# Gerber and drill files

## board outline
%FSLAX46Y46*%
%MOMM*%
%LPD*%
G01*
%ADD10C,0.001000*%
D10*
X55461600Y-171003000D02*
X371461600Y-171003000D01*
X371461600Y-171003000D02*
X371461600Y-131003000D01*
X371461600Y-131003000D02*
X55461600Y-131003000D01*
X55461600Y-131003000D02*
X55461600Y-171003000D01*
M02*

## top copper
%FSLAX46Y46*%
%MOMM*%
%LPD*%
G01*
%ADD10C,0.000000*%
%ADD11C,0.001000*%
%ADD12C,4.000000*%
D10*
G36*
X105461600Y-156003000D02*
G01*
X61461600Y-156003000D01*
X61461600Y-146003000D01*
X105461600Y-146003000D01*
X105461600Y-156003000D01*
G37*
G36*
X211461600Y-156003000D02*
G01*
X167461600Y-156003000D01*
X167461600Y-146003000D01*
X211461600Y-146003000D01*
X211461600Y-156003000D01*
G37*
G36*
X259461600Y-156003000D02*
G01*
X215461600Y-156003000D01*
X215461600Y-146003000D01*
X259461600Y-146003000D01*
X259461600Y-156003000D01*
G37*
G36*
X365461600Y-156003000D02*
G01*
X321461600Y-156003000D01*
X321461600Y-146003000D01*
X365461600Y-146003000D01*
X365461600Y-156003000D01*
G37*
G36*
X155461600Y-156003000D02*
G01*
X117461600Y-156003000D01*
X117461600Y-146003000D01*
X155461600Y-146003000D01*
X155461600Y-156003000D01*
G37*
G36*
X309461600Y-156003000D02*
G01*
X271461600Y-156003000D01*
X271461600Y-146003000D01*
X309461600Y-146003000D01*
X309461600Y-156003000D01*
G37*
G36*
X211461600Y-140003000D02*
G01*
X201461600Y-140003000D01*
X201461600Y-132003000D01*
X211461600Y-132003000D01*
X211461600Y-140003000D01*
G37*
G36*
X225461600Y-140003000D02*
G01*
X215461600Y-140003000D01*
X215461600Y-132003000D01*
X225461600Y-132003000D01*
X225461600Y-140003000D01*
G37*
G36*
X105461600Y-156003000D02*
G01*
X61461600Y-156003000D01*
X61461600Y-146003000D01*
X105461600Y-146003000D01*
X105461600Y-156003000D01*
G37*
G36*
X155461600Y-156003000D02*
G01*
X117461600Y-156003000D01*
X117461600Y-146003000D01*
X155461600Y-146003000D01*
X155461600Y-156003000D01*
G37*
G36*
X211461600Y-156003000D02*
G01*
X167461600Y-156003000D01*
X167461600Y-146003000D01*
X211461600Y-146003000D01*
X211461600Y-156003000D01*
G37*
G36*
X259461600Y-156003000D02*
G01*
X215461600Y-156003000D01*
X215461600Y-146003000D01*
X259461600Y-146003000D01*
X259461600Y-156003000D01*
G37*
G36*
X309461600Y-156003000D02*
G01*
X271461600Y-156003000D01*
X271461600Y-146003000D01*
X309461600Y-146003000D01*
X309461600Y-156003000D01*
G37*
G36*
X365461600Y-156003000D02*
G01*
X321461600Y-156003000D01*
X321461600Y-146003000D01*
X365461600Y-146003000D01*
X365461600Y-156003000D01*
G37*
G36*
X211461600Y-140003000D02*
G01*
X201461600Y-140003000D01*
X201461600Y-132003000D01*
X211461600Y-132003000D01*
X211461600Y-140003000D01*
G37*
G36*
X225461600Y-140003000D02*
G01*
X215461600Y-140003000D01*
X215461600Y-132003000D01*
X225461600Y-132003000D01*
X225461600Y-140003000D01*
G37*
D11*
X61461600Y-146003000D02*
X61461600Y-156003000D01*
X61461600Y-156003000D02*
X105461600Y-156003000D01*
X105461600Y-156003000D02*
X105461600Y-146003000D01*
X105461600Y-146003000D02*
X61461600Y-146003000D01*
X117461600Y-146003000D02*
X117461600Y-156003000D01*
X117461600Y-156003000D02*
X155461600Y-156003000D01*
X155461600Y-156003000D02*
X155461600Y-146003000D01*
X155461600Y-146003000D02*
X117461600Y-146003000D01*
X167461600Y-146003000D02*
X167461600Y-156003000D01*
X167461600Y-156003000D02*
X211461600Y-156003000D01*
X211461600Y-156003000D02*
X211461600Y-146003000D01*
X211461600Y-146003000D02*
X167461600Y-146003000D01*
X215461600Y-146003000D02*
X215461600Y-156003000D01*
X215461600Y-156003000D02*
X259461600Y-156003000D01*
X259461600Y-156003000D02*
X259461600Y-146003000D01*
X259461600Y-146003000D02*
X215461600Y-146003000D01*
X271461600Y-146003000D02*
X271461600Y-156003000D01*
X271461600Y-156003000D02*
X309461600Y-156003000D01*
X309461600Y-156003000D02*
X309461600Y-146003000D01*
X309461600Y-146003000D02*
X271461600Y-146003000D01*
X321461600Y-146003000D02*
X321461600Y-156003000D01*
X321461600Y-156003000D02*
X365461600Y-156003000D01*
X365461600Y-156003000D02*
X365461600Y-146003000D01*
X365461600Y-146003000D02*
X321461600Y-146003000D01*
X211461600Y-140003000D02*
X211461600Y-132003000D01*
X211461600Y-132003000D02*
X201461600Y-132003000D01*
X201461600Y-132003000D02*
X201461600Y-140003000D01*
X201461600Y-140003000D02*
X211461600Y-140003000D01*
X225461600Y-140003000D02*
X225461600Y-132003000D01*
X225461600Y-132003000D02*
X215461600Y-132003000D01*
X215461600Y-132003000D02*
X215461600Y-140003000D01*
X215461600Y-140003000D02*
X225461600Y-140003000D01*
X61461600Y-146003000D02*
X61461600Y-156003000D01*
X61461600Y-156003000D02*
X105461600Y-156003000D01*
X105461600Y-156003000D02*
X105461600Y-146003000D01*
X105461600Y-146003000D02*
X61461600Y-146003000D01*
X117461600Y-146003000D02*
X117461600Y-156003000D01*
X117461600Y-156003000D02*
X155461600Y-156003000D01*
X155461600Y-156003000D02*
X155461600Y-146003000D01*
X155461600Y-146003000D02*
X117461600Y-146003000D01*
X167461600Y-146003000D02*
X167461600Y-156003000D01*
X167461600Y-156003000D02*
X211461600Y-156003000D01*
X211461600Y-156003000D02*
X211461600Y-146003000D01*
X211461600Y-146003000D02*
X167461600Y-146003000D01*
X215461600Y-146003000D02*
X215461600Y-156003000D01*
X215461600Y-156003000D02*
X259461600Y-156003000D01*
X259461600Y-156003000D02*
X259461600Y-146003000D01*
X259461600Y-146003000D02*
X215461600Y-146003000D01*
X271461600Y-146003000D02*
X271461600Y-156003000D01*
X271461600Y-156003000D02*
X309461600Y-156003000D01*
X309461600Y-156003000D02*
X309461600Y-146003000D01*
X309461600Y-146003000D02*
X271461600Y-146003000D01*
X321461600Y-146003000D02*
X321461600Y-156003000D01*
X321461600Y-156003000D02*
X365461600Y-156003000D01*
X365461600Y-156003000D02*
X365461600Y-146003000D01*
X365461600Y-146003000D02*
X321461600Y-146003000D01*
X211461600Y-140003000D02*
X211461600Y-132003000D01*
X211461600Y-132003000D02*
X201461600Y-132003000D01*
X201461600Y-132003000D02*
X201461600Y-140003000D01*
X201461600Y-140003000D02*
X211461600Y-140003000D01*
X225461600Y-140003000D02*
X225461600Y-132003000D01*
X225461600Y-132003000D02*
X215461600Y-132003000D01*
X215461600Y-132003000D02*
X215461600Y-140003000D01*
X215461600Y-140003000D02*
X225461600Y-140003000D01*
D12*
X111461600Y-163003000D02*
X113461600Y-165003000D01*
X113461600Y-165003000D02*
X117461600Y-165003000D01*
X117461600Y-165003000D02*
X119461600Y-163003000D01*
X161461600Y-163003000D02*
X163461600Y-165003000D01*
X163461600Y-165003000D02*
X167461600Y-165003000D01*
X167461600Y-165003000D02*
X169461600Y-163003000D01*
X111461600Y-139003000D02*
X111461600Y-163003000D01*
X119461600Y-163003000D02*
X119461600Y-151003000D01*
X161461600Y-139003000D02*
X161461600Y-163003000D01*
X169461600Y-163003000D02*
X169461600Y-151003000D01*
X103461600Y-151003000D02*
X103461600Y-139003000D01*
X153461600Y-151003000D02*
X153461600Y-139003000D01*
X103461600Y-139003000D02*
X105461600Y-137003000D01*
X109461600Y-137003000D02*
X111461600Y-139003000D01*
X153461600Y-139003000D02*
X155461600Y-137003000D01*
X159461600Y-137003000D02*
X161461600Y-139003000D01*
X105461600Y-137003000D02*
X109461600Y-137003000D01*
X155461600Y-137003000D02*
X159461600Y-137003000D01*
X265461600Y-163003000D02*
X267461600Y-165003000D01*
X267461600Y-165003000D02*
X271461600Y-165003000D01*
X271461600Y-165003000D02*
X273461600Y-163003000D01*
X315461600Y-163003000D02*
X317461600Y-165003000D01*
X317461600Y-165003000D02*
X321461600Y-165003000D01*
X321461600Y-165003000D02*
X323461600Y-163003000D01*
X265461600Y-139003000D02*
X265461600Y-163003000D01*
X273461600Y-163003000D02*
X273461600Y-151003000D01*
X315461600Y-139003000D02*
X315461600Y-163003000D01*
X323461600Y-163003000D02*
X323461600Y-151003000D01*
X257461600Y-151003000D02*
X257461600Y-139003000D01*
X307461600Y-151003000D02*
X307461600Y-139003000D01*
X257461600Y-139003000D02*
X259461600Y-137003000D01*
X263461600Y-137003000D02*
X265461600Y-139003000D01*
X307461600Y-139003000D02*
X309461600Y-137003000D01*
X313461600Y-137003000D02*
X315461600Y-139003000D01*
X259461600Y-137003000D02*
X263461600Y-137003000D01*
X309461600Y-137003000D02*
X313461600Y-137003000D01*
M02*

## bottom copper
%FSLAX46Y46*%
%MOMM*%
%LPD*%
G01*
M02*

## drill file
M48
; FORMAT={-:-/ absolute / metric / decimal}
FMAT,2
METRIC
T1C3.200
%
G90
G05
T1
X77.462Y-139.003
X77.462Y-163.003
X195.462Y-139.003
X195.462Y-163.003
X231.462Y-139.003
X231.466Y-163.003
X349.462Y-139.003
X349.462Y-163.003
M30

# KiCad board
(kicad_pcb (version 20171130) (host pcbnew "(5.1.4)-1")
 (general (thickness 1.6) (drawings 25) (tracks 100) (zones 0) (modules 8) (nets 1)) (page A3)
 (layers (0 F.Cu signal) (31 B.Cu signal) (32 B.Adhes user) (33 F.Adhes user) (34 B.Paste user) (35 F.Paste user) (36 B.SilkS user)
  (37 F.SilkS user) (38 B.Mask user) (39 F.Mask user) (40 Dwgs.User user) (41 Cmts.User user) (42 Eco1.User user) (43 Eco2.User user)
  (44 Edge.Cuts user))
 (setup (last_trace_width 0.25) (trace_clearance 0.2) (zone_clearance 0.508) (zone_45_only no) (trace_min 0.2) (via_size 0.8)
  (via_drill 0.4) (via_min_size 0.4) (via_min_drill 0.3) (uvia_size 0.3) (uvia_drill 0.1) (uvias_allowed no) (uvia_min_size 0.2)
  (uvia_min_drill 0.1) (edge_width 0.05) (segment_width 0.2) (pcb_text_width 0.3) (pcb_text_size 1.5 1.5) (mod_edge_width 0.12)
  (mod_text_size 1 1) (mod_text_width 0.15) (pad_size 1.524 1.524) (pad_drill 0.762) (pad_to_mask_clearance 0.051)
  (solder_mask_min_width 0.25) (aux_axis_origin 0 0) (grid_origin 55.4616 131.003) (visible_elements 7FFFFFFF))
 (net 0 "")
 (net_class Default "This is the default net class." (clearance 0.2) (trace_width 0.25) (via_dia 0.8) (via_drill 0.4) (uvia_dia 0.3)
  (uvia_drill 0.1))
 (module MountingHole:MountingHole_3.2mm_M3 (layer F.Cu) (at 349.4616 139.003)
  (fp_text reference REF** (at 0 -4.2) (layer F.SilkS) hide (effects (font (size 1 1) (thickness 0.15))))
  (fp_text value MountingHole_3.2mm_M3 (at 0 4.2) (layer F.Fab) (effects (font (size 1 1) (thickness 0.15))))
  (pad 1 np_thru_hole circle (at 0 0) (size 3.2 3.2) (drill 3.2) (layers *.Cu *.Mask)))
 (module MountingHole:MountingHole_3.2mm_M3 (layer F.Cu) (at 349.4616 163.003)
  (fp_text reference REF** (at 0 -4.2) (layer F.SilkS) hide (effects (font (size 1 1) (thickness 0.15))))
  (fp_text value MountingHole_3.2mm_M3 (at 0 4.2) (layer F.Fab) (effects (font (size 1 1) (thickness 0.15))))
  (pad 1 np_thru_hole circle (at 0 0) (size 3.2 3.2) (drill 3.2) (layers *.Cu *.Mask)))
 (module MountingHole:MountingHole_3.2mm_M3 (layer F.Cu) (at 195.4616 139.003)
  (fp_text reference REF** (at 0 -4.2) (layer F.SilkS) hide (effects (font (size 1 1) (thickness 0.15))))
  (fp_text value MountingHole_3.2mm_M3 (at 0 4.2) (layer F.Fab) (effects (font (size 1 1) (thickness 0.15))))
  (pad 1 np_thru_hole circle (at 0 0) (size 3.2 3.2) (drill 3.2) (layers *.Cu *.Mask)))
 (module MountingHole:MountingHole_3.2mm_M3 (layer F.Cu) (at 231.4616 139.003)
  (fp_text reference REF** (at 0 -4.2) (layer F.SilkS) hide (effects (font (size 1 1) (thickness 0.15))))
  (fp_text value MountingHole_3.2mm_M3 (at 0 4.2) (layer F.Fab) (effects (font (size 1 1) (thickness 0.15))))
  (pad 1 np_thru_hole circle (at 0 0) (size 3.2 3.2) (drill 3.2) (layers *.Cu *.Mask)))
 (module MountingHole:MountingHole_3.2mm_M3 (layer F.Cu) (at 231.4661 163.003)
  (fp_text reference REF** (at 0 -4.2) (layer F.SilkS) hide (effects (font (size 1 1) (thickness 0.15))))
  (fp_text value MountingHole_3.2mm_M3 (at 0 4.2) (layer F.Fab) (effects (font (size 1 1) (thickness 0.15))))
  (pad 1 np_thru_hole circle (at 0 0) (size 3.2 3.2) (drill 3.2) (layers *.Cu *.Mask)))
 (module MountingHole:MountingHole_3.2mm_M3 (layer F.Cu) (at 195.4616 163.003)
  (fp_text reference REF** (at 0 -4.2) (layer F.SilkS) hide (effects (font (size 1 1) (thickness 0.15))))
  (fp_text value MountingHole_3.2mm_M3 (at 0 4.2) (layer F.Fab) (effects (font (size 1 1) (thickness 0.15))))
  (pad 1 np_thru_hole circle (at 0 0) (size 3.2 3.2) (drill 3.2) (layers *.Cu *.Mask)))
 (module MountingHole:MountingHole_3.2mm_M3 (layer F.Cu) (at 77.4616 163.003)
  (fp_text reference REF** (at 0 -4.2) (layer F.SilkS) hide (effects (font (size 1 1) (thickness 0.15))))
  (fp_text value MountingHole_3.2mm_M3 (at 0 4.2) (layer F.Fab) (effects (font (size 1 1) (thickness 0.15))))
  (pad 1 np_thru_hole circle (at 0 0) (size 3.2 3.2) (drill 3.2) (layers *.Cu *.Mask)))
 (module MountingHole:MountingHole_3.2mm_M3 (layer F.Cu) (at 77.4616 139.003)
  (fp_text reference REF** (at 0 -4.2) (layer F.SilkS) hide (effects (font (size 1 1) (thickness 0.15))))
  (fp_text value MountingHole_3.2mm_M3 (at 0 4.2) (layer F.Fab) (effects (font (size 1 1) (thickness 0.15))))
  (pad 1 np_thru_hole circle (at 0 0) (size 3.2 3.2) (drill 3.2) (layers *.Cu *.Mask)))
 (gr_line (start 55.4616 171.003) (end 371.4616 171.003) (layer Edge.Cuts) (width 0.001))
 (gr_line (start 371.4616 171.003) (end 371.4616 131.003) (layer Edge.Cuts) (width 0.001))
 (gr_line (start 371.4616 131.003) (end 55.4616 131.003) (layer Edge.Cuts) (width 0.001))
 (gr_line (start 55.4616 131.003) (end 55.4616 171.003) (layer Edge.Cuts) (width 0.001))
 (gr_poly (pts (xy 61.4616 146.003) (xy 61.4616 156.003) (xy 105.4616 156.003) (xy 105.4616 146.003)) (layer F.Cu) (width 0))
 (gr_poly (pts (xy 167.4616 146.003) (xy 167.4616 156.003) (xy 211.4616 156.003) (xy 211.4616 146.003)) (layer F.Cu) (width 0))
 (gr_poly (pts (xy 215.4616 146.003) (xy 215.4616 156.003) (xy 259.4616 156.003) (xy 259.4616 146.003)) (layer F.Cu) (width 0))
 (gr_poly (pts (xy 321.4616 146.003) (xy 321.4616 156.003) (xy 365.4616 156.003) (xy 365.4616 146.003)) (layer F.Cu) (width 0))
 (gr_poly (pts (xy 117.4616 146.003) (xy 117.4616 156.003) (xy 155.4616 156.003) (xy 155.4616 146.003)) (layer F.Cu) (width 0))
 (gr_poly (pts (xy 271.4616 146.003) (xy 271.4616 156.003) (xy 309.4616 156.003) (xy 309.4616 146.003)) (layer F.Cu) (width 0))
 (gr_poly (pts (xy 211.4616 140.003) (xy 211.4616 132.003) (xy 201.4616 132.003) (xy 201.4616 140.003)) (layer F.Cu) (width 0))
 (gr_poly (pts (xy 225.4616 140.003) (xy 225.4616 132.003) (xy 215.4616 132.003) (xy 215.4616 140.003)) (layer F.Cu) (width 0))
 (gr_poly (pts (xy 61.4616 146.003) (xy 61.4616 156.003) (xy 105.4616 156.003) (xy 105.4616 146.003)) (layer F.Cu) (width 0))
 (gr_poly (pts (xy 117.4616 146.003) (xy 117.4616 156.003) (xy 155.4616 156.003) (xy 155.4616 146.003)) (layer F.Cu) (width 0))
 (gr_poly (pts (xy 167.4616 146.003) (xy 167.4616 156.003) (xy 211.4616 156.003) (xy 211.4616 146.003)) (layer F.Cu) (width 0))
 (gr_poly (pts (xy 215.4616 146.003) (xy 215.4616 156.003) (xy 259.4616 156.003) (xy 259.4616 146.003)) (layer F.Cu) (width 0))
 (gr_poly (pts (xy 271.4616 146.003) (xy 271.4616 156.003) (xy 309.4616 156.003) (xy 309.4616 146.003)) (layer F.Cu) (width 0))
 (gr_poly (pts (xy 321.4616 146.003) (xy 321.4616 156.003) (xy 365.4616 156.003) (xy 365.4616 146.003)) (layer F.Cu) (width 0))
 (gr_poly (pts (xy 211.4616 140.003) (xy 211.4616 132.003) (xy 201.4616 132.003) (xy 201.4616 140.003)) (layer F.Cu) (width 0))
 (gr_poly (pts (xy 225.4616 140.003) (xy 225.4616 132.003) (xy 215.4616 132.003) (xy 215.4616 140.003)) (layer F.Cu) (width 0))
 (segment (start 61.4616 146.003) (end 61.4616 156.003) (width 0.001) (layer F.Cu) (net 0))
 (segment (start 61.4616 156.003) (end 105.4616 156.003) (width 0.001) (layer F.Cu) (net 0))
 (segment (start 105.4616 156.003) (end 105.4616 146.003) (width 0.001) (layer F.Cu) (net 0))
 (segment (start 105.4616 146.003) (end 61.4616 146.003) (width 0.001) (layer F.Cu) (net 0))
 (segment (start 117.4616 146.003) (end 117.4616 156.003) (width 0.001) (layer F.Cu) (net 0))
 (segment (start 117.4616 156.003) (end 155.4616 156.003) (width 0.001) (layer F.Cu) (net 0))
 (segment (start 155.4616 156.003) (end 155.4616 146.003) (width 0.001) (layer F.Cu) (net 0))
 (segment (start 155.4616 146.003) (end 117.4616 146.003) (width 0.001) (layer F.Cu) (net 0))
 (segment (start 167.4616 146.003) (end 167.4616 156.003) (width 0.001) (layer F.Cu) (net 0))
 (segment (start 167.4616 156.003) (end 211.4616 156.003) (width 0.001) (layer F.Cu) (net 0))
 (segment (start 211.4616 156.003) (end 211.4616 146.003) (width 0.001) (layer F.Cu) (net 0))
 (segment (start 211.4616 146.003) (end 167.4616 146.003) (width 0.001) (layer F.Cu) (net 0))
 (segment (start 215.4616 146.003) (end 215.4616 156.003) (width 0.001) (layer F.Cu) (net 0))
 (segment (start 215.4616 156.003) (end 259.4616 156.003) (width 0.001) (layer F.Cu) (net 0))
 (segment (start 259.4616 156.003) (end 259.4616 146.003) (width 0.001) (layer F.Cu) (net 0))
 (segment (start 259.4616 146.003) (end 215.4616 146.003) (width 0.001) (layer F.Cu) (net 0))
 (segment (start 271.4616 146.003) (end 271.4616 156.003) (width 0.001) (layer F.Cu) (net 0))
 (segment (start 271.4616 156.003) (end 309.4616 156.003) (width 0.001) (layer F.Cu) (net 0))
 (segment (start 309.4616 156.003) (end 309.4616 146.003) (width 0.001) (layer F.Cu) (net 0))
 (segment (start 309.4616 146.003) (end 271.4616 146.003) (width 0.001) (layer F.Cu) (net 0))
 (segment (start 321.4616 146.003) (end 321.4616 156.003) (width 0.001) (layer F.Cu) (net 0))
 (segment (start 321.4616 156.003) (end 365.4616 156.003) (width 0.001) (layer F.Cu) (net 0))
 (segment (start 365.4616 156.003) (end 365.4616 146.003) (width 0.001) (layer F.Cu) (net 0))
 (segment (start 365.4616 146.003) (end 321.4616 146.003) (width 0.001) (layer F.Cu) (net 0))
 (segment (start 211.4616 140.003) (end 211.4616 132.003) (width 0.001) (layer F.Cu) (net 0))
 (segment (start 211.4616 132.003) (end 201.4616 132.003) (width 0.001) (layer F.Cu) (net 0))
 (segment (start 201.4616 132.003) (end 201.4616 140.003) (width 0.001) (layer F.Cu) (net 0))
 (segment (start 201.4616 140.003) (end 211.4616 140.003) (width 0.001) (layer F.Cu) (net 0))
 (segment (start 225.4616 140.003) (end 225.4616 132.003) (width 0.001) (layer F.Cu) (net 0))
 (segment (start 225.4616 132.003) (end 215.4616 132.003) (width 0.001) (layer F.Cu) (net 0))
 (segment (start 215.4616 132.003) (end 215.4616 140.003) (width 0.001) (layer F.Cu) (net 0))
 (segment (start 215.4616 140.003) (end 225.4616 140.003) (width 0.001) (layer F.Cu) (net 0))
 (segment (start 61.4616 146.003) (end 61.4616 156.003) (width 0.001) (layer F.Cu) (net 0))
 (segment (start 61.4616 156.003) (end 105.4616 156.003) (width 0.001) (layer F.Cu) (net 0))
 (segment (start 105.4616 156.003) (end 105.4616 146.003) (width 0.001) (layer F.Cu) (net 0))
 (segment (start 105.4616 146.003) (end 61.4616 146.003) (width 0.001) (layer F.Cu) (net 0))
 (segment (start 117.4616 146.003) (end 117.4616 156.003) (width 0.001) (layer F.Cu) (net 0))
 (segment (start 117.4616 156.003) (end 155.4616 156.003) (width 0.001) (layer F.Cu) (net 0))
 (segment (start 155.4616 156.003) (end 155.4616 146.003) (width 0.001) (layer F.Cu) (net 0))
 (segment (start 155.4616 146.003) (end 117.4616 146.003) (width 0.001) (layer F.Cu) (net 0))
 (segment (start 167.4616 146.003) (end 167.4616 156.003) (width 0.001) (layer F.Cu) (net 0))
 (segment (start 167.4616 156.003) (end 211.4616 156.003) (width 0.001) (layer F.Cu) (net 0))
 (segment (start 211.4616 156.003) (end 211.4616 146.003) (width 0.001) (layer F.Cu) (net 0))
 (segment (start 211.4616 146.003) (end 167.4616 146.003) (width 0.001) (layer F.Cu) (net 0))
 (segment (start 215.4616 146.003) (end 215.4616 156.003) (width 0.001) (layer F.Cu) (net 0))
 (segment (start 215.4616 156.003) (end 259.4616 156.003) (width 0.001) (layer F.Cu) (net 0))
 (segment (start 259.4616 156.003) (end 259.4616 146.003) (width 0.001) (layer F.Cu) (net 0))
 (segment (start 259.4616 146.003) (end 215.4616 146.003) (width 0.001) (layer F.Cu) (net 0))
 (segment (start 271.4616 146.003) (end 271.4616 156.003) (width 0.001) (layer F.Cu) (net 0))
 (segment (start 271.4616 156.003) (end 309.4616 156.003) (width 0.001) (layer F.Cu) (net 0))
 (segment (start 309.4616 156.003) (end 309.4616 146.003) (width 0.001) (layer F.Cu) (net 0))
 (segment (start 309.4616 146.003) (end 271.4616 146.003) (width 0.001) (layer F.Cu) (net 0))
 (segment (start 321.4616 146.003) (end 321.4616 156.003) (width 0.001) (layer F.Cu) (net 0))
 (segment (start 321.4616 156.003) (end 365.4616 156.003) (width 0.001) (layer F.Cu) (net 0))
 (segment (start 365.4616 156.003) (end 365.4616 146.003) (width 0.001) (layer F.Cu) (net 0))
 (segment (start 365.4616 146.003) (end 321.4616 146.003) (width 0.001) (layer F.Cu) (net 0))
 (segment (start 211.4616 140.003) (end 211.4616 132.003) (width 0.001) (layer F.Cu) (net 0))
 (segment (start 211.4616 132.003) (end 201.4616 132.003) (width 0.001) (layer F.Cu) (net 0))
 (segment (start 201.4616 132.003) (end 201.4616 140.003) (width 0.001) (layer F.Cu) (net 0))
 (segment (start 201.4616 140.003) (end 211.4616 140.003) (width 0.001) (layer F.Cu) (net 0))
 (segment (start 225.4616 140.003) (end 225.4616 132.003) (width 0.001) (layer F.Cu) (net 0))
 (segment (start 225.4616 132.003) (end 215.4616 132.003) (width 0.001) (layer F.Cu) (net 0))
 (segment (start 215.4616 132.003) (end 215.4616 140.003) (width 0.001) (layer F.Cu) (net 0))
 (segment (start 215.4616 140.003) (end 225.4616 140.003) (width 0.001) (layer F.Cu) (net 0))
 (segment (start 111.4616 163.003) (end 113.4616 165.003) (width 4) (layer F.Cu) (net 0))
 (segment (start 113.4616 165.003) (end 117.4616 165.003) (width 4) (layer F.Cu) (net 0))
 (segment (start 117.4616 165.003) (end 119.4616 163.003) (width 4) (layer F.Cu) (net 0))
 (segment (start 161.4616 163.003) (end 163.4616 165.003) (width 4) (layer F.Cu) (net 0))
 (segment (start 163.4616 165.003) (end 167.4616 165.003) (width 4) (layer F.Cu) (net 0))
 (segment (start 167.4616 165.003) (end 169.4616 163.003) (width 4) (layer F.Cu) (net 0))
 (segment (start 111.4616 139.003) (end 111.4616 163.003) (width 4) (layer F.Cu) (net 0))
 (segment (start 119.4616 163.003) (end 119.4616 151.003) (width 4) (layer F.Cu) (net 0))
 (segment (start 161.4616 139.003) (end 161.4616 163.003) (width 4) (layer F.Cu) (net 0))
 (segment (start 169.4616 163.003) (end 169.4616 151.003) (width 4) (layer F.Cu) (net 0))
 (segment (start 103.4616 151.003) (end 103.4616 139.003) (width 4) (layer F.Cu) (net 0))
 (segment (start 153.4616 151.003) (end 153.4616 139.003) (width 4) (layer F.Cu) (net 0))
 (segment (start 103.4616 139.003) (end 105.4616 137.003) (width 4) (layer F.Cu) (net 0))
 (segment (start 109.4616 137.003) (end 111.4616 139.003) (width 4) (layer F.Cu) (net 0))
 (segment (start 153.4616 139.003) (end 155.4616 137.003) (width 4) (layer F.Cu) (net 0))
 (segment (start 159.4616 137.003) (end 161.4616 139.003) (width 4) (layer F.Cu) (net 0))
 (segment (start 105.4616 137.003) (end 109.4616 137.003) (width 4) (layer F.Cu) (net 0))
 (segment (start 155.4616 137.003) (end 159.4616 137.003) (width 4) (layer F.Cu) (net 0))
 (segment (start 265.4616 163.003) (end 267.4616 165.003) (width 4) (layer F.Cu) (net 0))
 (segment (start 267.4616 165.003) (end 271.4616 165.003) (width 4) (layer F.Cu) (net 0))
 (segment (start 271.4616 165.003) (end 273.4616 163.003) (width 4) (layer F.Cu) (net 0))
 (segment (start 315.4616 163.003) (end 317.4616 165.003) (width 4) (layer F.Cu) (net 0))
 (segment (start 317.4616 165.003) (end 321.4616 165.003) (width 4) (layer F.Cu) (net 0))
 (segment (start 321.4616 165.003) (end 323.4616 163.003) (width 4) (layer F.Cu) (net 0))
 (segment (start 265.4616 139.003) (end 265.4616 163.003) (width 4) (layer F.Cu) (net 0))
 (segment (start 273.4616 163.003) (end 273.4616 151.003) (width 4) (layer F.Cu) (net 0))
 (segment (start 315.4616 139.003) (end 315.4616 163.003) (width 4) (layer F.Cu) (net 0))
 (segment (start 323.4616 163.003) (end 323.4616 151.003) (width 4) (layer F.Cu) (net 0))
 (segment (start 257.4616 151.003) (end 257.4616 139.003) (width 4) (layer F.Cu) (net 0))
 (segment (start 307.4616 151.003) (end 307.4616 139.003) (width 4) (layer F.Cu) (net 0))
 (segment (start 257.4616 139.003) (end 259.4616 137.003) (width 4) (layer F.Cu) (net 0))
 (segment (start 263.4616 137.003) (end 265.4616 139.003) (width 4) (layer F.Cu) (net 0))
 (segment (start 307.4616 139.003) (end 309.4616 137.003) (width 4) (layer F.Cu) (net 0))
 (segment (start 313.4616 137.003) (end 315.4616 139.003) (width 4) (layer F.Cu) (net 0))
 (segment (start 259.4616 137.003) (end 263.4616 137.003) (width 4) (layer F.Cu) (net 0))
 (segment (start 309.4616 137.003) (end 313.4616 137.003) (width 4) (layer F.Cu) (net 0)))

